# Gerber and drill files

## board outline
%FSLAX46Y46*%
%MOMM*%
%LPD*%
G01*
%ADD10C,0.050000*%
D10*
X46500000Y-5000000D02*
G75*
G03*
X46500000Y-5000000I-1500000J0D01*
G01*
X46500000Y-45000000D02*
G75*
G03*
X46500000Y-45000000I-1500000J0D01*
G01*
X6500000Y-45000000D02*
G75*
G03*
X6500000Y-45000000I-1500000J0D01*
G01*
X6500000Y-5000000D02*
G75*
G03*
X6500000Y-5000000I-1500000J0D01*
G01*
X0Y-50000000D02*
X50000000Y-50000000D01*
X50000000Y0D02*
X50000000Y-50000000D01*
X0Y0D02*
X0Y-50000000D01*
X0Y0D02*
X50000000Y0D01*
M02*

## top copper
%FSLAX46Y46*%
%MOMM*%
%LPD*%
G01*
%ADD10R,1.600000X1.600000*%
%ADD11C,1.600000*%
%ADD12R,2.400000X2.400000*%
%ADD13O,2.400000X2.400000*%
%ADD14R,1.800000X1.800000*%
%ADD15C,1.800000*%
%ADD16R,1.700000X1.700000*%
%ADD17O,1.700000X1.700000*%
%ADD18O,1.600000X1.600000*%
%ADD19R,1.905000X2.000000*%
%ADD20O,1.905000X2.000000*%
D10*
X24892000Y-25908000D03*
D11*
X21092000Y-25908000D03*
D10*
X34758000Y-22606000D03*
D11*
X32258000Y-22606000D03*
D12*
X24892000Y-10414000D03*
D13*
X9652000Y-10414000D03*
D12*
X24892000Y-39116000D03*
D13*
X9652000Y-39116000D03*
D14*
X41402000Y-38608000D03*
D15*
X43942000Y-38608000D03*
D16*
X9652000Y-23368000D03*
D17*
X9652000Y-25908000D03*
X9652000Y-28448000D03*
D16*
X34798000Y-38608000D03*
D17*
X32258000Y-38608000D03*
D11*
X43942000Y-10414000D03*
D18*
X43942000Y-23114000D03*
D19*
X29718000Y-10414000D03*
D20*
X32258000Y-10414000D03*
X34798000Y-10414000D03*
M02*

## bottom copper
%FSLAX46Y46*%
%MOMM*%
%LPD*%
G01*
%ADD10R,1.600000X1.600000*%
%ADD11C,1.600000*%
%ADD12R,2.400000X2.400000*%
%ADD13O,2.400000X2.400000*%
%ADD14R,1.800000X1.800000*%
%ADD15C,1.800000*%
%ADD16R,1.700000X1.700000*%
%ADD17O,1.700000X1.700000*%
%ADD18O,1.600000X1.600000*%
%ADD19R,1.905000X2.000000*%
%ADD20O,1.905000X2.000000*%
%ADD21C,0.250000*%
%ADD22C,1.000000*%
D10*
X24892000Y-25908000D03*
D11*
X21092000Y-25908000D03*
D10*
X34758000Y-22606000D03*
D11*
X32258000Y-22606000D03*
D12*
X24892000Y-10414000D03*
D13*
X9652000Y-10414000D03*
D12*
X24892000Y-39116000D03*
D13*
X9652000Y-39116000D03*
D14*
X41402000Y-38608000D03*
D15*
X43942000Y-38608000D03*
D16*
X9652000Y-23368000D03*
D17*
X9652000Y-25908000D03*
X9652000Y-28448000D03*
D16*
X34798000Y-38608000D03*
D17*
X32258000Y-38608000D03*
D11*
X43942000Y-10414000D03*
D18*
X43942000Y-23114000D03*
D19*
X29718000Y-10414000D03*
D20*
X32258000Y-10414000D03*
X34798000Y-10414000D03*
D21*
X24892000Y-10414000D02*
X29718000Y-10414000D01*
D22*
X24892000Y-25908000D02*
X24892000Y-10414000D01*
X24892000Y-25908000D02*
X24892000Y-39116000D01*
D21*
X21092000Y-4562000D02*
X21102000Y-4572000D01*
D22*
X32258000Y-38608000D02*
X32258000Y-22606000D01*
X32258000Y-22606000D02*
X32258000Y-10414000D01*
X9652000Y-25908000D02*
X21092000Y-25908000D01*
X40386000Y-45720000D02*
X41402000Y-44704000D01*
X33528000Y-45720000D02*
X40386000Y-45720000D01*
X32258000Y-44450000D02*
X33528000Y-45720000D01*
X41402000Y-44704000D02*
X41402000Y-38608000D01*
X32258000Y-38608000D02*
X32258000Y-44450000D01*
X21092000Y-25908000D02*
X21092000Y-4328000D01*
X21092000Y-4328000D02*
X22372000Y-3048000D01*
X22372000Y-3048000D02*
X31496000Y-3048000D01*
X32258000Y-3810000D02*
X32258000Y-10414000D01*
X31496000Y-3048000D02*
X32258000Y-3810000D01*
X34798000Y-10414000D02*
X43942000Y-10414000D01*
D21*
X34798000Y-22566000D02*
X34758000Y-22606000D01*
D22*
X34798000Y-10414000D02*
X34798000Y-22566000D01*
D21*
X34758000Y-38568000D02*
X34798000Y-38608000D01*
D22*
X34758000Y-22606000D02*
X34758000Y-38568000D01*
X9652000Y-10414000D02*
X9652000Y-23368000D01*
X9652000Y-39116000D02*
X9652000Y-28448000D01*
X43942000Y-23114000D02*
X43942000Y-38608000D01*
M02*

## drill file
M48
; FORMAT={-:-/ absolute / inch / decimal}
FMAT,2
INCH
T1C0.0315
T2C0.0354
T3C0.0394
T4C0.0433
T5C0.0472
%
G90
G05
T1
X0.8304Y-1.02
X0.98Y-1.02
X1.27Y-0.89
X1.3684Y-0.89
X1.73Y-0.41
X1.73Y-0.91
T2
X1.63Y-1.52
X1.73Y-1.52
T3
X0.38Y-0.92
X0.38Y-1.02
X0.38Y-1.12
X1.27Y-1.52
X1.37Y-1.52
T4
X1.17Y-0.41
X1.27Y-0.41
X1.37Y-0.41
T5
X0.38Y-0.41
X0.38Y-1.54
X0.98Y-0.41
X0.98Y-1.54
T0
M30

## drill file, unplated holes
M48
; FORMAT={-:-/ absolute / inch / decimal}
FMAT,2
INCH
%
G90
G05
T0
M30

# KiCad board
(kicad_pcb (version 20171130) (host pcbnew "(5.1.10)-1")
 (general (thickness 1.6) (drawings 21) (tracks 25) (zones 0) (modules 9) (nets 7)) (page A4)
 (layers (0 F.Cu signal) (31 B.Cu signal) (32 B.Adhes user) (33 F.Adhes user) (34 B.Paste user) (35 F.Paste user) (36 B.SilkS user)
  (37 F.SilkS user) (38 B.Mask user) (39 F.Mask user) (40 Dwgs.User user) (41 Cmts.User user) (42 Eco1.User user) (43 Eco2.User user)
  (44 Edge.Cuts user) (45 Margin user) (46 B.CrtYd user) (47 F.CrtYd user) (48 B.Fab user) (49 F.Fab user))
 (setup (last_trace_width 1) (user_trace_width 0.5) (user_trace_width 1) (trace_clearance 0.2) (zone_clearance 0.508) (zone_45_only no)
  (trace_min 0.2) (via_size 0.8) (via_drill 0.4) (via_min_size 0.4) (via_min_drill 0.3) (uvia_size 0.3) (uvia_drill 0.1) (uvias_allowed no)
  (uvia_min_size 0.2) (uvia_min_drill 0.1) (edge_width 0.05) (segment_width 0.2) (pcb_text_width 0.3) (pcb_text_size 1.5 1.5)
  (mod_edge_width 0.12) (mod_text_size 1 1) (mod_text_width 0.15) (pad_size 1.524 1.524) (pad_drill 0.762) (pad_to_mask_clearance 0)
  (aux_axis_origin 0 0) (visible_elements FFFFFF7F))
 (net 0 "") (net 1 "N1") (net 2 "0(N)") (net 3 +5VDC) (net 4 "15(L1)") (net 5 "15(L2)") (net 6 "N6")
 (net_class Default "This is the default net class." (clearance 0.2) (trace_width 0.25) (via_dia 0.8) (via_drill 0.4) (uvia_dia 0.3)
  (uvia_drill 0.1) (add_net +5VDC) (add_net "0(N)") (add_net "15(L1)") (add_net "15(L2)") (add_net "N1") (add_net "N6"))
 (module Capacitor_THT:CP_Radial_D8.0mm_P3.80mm (layer F.Cu) (at 24.892 25.908 180)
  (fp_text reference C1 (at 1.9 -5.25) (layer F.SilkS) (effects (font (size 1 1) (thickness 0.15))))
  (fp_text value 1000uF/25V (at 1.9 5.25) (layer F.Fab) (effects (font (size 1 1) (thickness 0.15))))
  (pad 1 thru_hole rect (at 0 0 180) (size 1.6 1.6) (drill 0.8) (layers *.Cu *.Mask) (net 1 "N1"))
  (pad 2 thru_hole circle (at 3.8 0 180) (size 1.6 1.6) (drill 0.8) (layers *.Cu *.Mask) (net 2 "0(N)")))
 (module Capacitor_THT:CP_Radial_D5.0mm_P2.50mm (layer F.Cu) (at 34.758 22.606 180)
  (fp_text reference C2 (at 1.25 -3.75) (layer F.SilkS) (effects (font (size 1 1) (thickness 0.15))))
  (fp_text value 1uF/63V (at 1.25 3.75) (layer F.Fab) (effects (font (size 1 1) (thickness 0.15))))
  (pad 1 thru_hole rect (at 0 0 180) (size 1.6 1.6) (drill 0.8) (layers *.Cu *.Mask) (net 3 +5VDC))
  (pad 2 thru_hole circle (at 2.5 0 180) (size 1.6 1.6) (drill 0.8) (layers *.Cu *.Mask) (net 2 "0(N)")))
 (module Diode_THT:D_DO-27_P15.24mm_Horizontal (layer F.Cu) (at 24.892 10.414 180)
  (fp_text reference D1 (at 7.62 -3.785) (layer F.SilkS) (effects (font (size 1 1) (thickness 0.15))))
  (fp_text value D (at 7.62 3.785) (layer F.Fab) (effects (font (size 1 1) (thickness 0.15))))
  (pad 1 thru_hole rect (at 0 0 180) (size 2.4 2.4) (drill 1.2) (layers *.Cu *.Mask) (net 1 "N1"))
  (pad 2 thru_hole oval (at 15.24 0 180) (size 2.4 2.4) (drill 1.2) (layers *.Cu *.Mask) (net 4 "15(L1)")))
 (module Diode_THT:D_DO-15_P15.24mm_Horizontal (layer F.Cu) (at 24.892 39.116 180)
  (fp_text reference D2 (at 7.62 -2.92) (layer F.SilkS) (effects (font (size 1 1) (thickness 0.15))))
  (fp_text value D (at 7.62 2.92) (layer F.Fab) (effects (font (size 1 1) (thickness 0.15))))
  (pad 1 thru_hole rect (at 0 0 180) (size 2.4 2.4) (drill 1.2) (layers *.Cu *.Mask) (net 1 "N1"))
  (pad 2 thru_hole oval (at 15.24 0 180) (size 2.4 2.4) (drill 1.2) (layers *.Cu *.Mask) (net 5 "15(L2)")))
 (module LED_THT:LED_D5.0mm (layer F.Cu) (at 41.402 38.608)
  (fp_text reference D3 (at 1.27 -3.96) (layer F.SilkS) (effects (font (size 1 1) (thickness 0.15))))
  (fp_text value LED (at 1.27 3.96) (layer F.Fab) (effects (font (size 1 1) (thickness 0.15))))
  (pad 1 thru_hole rect (at 0 0) (size 1.8 1.8) (drill 0.9) (layers *.Cu *.Mask) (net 2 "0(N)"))
  (pad 2 thru_hole circle (at 2.54 0) (size 1.8 1.8) (drill 0.9) (layers *.Cu *.Mask) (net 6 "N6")))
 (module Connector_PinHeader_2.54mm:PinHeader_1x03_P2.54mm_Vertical (layer F.Cu) (at 9.652 23.368)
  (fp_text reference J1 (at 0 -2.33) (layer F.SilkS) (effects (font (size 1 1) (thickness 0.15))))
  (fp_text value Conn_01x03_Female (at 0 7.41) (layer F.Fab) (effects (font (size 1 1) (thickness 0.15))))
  (pad 1 thru_hole rect (at 0 0) (size 1.7 1.7) (drill 1) (layers *.Cu *.Mask) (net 4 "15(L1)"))
  (pad 2 thru_hole oval (at 0 2.54) (size 1.7 1.7) (drill 1) (layers *.Cu *.Mask) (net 2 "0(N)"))
  (pad 3 thru_hole oval (at 0 5.08) (size 1.7 1.7) (drill 1) (layers *.Cu *.Mask) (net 5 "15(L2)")))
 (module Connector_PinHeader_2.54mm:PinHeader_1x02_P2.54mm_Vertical (layer F.Cu) (at 34.798 38.608 270)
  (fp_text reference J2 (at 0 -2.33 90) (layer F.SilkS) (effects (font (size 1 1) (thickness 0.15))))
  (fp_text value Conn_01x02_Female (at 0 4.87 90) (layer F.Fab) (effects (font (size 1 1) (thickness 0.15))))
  (pad 1 thru_hole rect (at 0 0 270) (size 1.7 1.7) (drill 1) (layers *.Cu *.Mask) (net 3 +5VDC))
  (pad 2 thru_hole oval (at 0 2.54 270) (size 1.7 1.7) (drill 1) (layers *.Cu *.Mask) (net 2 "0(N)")))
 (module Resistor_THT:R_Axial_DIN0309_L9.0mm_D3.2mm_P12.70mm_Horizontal (layer F.Cu) (at 43.942 10.414 270)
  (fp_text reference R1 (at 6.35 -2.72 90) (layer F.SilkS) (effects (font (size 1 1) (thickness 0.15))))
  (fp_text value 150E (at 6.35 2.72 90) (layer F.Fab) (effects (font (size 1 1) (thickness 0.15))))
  (pad 1 thru_hole circle (at 0 0 270) (size 1.6 1.6) (drill 0.8) (layers *.Cu *.Mask) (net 3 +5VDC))
  (pad 2 thru_hole oval (at 12.7 0 270) (size 1.6 1.6) (drill 0.8) (layers *.Cu *.Mask) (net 6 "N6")))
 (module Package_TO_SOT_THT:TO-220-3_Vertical (layer F.Cu) (at 29.718 10.414)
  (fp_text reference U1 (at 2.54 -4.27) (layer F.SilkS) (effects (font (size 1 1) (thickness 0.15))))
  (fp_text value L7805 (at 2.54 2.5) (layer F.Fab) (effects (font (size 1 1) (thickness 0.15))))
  (pad 1 thru_hole rect (at 0 0) (size 1.905 2) (drill 1.1) (layers *.Cu *.Mask) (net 1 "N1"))
  (pad 2 thru_hole oval (at 2.54 0) (size 1.905 2) (drill 1.1) (layers *.Cu *.Mask) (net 2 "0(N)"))
  (pad 3 thru_hole oval (at 5.08 0) (size 1.905 2) (drill 1.1) (layers *.Cu *.Mask) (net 3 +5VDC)))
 (gr_circle (center 45 5) (end 46.5 5) (layer Edge.Cuts) (width 0.05))
 (gr_circle (center 45 45) (end 46.5 45) (layer Edge.Cuts) (width 0.05))
 (gr_circle (center 5 45) (end 6.5 45) (layer Edge.Cuts) (width 0.05))
 (gr_circle (center 5 5) (end 6.5 5) (layer Edge.Cuts) (width 0.05))
 (gr_line (start 0 50) (end 50 50) (layer Edge.Cuts) (width 0.05))
 (gr_line (start 50 0) (end 50 50) (layer Edge.Cuts) (width 0.05))
 (gr_line (start 0 0) (end 0 50) (layer Edge.Cuts) (width 0.05))
 (gr_line (start 0 0) (end 50 0) (layer Edge.Cuts) (width 0.05))
 (segment (start 24.892 10.414) (end 29.718 10.414) (width 1) (layer B.Cu) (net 1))
 (segment (start 24.892 25.908) (end 24.892 10.414) (width 1) (layer B.Cu) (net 1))
 (segment (start 24.892 25.908) (end 24.892 39.116) (width 1) (layer B.Cu) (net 1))
 (segment (start 21.092 4.562) (end 21.102 4.572) (width 0.25) (layer B.Cu) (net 2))
 (segment (start 32.258 38.608) (end 32.258 22.606) (width 1) (layer B.Cu) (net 2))
 (segment (start 32.258 22.606) (end 32.258 10.414) (width 1) (layer B.Cu) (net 2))
 (segment (start 9.652 25.908) (end 21.092 25.908) (width 1) (layer B.Cu) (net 2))
 (segment (start 40.386 45.72) (end 41.402 44.704) (width 1) (layer B.Cu) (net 2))
 (segment (start 33.528 45.72) (end 40.386 45.72) (width 1) (layer B.Cu) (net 2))
 (segment (start 32.258 44.45) (end 33.528 45.72) (width 1) (layer B.Cu) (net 2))
 (segment (start 41.402 44.704) (end 41.402 38.608) (width 1) (layer B.Cu) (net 2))
 (segment (start 32.258 38.608) (end 32.258 44.45) (width 1) (layer B.Cu) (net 2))
 (segment (start 21.092 25.908) (end 21.092 4.328) (width 1) (layer B.Cu) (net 2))
 (segment (start 21.092 4.328) (end 22.372 3.048) (width 1) (layer B.Cu) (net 2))
 (segment (start 22.372 3.048) (end 31.496 3.048) (width 1) (layer B.Cu) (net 2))
 (segment (start 32.258 3.81) (end 32.258 10.414) (width 1) (layer B.Cu) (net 2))
 (segment (start 31.496 3.048) (end 32.258 3.81) (width 1) (layer B.Cu) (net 2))
 (segment (start 34.798 10.414) (end 43.942 10.414) (width 1) (layer B.Cu) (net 3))
 (segment (start 34.798 22.566) (end 34.758 22.606) (width 0.25) (layer B.Cu) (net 3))
 (segment (start 34.798 10.414) (end 34.798 22.566) (width 1) (layer B.Cu) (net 3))
 (segment (start 34.758 38.568) (end 34.798 38.608) (width 0.25) (layer B.Cu) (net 3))
 (segment (start 34.758 22.606) (end 34.758 38.568) (width 1) (layer B.Cu) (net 3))
 (segment (start 9.652 10.414) (end 9.652 23.368) (width 1) (layer B.Cu) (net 4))
 (segment (start 9.652 39.116) (end 9.652 28.448) (width 1) (layer B.Cu) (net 5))
 (segment (start 43.942 23.114) (end 43.942 38.608) (width 1) (layer B.Cu) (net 6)))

